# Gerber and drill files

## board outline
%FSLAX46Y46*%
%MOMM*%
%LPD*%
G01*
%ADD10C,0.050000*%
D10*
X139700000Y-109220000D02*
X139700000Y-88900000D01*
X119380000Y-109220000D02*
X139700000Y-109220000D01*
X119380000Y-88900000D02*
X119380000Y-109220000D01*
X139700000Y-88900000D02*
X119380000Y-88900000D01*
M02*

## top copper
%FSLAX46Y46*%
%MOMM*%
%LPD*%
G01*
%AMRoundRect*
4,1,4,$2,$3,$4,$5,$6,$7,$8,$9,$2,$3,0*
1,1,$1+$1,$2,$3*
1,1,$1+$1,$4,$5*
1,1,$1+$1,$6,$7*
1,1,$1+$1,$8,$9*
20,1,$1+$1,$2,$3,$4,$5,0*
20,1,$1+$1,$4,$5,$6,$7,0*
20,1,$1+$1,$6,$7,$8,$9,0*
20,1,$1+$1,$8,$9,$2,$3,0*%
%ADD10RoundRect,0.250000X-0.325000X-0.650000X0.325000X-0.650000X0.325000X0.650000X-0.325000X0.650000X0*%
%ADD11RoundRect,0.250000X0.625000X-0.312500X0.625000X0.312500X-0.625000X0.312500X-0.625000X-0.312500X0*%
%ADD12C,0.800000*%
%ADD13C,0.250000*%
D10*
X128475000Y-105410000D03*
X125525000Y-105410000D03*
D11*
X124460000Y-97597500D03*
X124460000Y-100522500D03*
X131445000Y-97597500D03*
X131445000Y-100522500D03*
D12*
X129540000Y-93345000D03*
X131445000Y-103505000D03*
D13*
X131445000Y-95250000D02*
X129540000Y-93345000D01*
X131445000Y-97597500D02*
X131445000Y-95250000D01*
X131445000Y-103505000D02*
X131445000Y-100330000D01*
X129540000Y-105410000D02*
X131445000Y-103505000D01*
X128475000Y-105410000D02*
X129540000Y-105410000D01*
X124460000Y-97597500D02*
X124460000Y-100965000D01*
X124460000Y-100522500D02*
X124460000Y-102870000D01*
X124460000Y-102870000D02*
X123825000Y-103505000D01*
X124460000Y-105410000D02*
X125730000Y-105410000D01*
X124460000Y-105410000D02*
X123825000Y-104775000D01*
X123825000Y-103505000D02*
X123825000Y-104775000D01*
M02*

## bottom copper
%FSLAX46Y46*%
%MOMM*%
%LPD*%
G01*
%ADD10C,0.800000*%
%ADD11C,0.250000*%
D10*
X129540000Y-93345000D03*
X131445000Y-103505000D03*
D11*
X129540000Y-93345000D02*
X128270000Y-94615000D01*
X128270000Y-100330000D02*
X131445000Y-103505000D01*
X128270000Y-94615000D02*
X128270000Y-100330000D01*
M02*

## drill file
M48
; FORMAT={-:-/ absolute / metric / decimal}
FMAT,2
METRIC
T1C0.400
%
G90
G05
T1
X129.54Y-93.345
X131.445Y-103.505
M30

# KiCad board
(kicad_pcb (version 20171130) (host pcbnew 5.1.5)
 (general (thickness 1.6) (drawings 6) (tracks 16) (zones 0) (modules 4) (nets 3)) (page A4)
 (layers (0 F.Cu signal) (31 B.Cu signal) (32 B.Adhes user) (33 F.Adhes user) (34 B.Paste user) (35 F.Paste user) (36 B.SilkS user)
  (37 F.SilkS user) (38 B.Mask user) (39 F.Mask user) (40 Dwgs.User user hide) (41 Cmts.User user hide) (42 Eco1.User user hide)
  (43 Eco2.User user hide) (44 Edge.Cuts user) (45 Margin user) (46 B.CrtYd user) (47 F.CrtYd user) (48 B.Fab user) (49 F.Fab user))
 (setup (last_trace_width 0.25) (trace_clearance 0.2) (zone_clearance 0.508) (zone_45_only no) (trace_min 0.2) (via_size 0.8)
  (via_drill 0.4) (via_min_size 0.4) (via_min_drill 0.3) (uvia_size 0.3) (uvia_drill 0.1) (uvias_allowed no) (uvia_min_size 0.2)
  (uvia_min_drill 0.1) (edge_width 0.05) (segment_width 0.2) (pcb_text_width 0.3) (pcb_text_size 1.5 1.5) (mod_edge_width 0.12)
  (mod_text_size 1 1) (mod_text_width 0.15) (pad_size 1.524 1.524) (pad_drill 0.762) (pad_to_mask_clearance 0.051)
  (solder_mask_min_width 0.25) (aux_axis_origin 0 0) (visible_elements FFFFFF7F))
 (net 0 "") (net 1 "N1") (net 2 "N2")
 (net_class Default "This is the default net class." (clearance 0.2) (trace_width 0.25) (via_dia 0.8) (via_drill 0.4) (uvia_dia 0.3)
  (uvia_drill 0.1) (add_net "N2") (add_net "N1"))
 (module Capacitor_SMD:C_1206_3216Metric (layer F.Cu) (at 127 105.41)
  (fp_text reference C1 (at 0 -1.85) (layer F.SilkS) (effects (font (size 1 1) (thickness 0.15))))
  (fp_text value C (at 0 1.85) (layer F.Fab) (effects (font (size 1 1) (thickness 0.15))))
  (pad 2 smd roundrect (at 1.475 0) (size 1.15 1.8) (layers F.Cu F.Paste F.Mask) (roundrect_rratio 0.217391) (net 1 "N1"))
  (pad 1 smd roundrect (at -1.475 0) (size 1.15 1.8) (layers F.Cu F.Paste F.Mask) (roundrect_rratio 0.217391) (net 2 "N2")))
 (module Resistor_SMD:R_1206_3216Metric (layer F.Cu) (at 124.46 99.06 90)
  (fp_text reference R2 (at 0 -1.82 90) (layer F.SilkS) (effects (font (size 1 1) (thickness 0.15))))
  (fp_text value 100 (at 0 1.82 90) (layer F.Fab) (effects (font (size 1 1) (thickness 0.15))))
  (pad 2 smd roundrect (at 1.4625 0 90) (size 1.125 1.75) (layers F.Cu F.Paste F.Mask) (roundrect_rratio 0.222222) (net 2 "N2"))
  (pad 1 smd roundrect (at -1.4625 0 90) (size 1.125 1.75) (layers F.Cu F.Paste F.Mask) (roundrect_rratio 0.222222) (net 2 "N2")))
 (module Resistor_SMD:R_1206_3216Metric (layer F.Cu) (at 131.445 99.06 90)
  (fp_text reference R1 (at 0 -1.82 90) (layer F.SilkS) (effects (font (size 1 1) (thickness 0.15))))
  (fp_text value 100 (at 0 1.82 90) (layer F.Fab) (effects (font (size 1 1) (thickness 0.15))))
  (pad 2 smd roundrect (at 1.4625 0 90) (size 1.125 1.75) (layers F.Cu F.Paste F.Mask) (roundrect_rratio 0.222222) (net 1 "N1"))
  (pad 1 smd roundrect (at -1.4625 0 90) (size 1.125 1.75) (layers F.Cu F.Paste F.Mask) (roundrect_rratio 0.222222) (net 1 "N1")))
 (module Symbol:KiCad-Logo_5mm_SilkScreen (layer F.Cu) (at 137.795 95.25 90)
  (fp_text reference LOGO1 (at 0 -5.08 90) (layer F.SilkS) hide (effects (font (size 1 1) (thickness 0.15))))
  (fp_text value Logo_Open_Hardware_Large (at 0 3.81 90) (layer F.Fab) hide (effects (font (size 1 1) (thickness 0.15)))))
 (gr_line (start 139.7 109.22) (end 139.7 88.9) (layer Edge.Cuts) (width 0.05))
 (gr_line (start 119.38 109.22) (end 139.7 109.22) (layer Edge.Cuts) (width 0.05))
 (gr_line (start 119.38 88.9) (end 119.38 109.22) (layer Edge.Cuts) (width 0.05))
 (gr_line (start 139.7 88.9) (end 119.38 88.9) (layer Edge.Cuts) (width 0.05))
 (via (at 129.54 93.345) (size 0.8) (drill 0.4) (layers F.Cu B.Cu) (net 1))
 (segment (start 131.445 95.25) (end 129.54 93.345) (width 0.25) (layer F.Cu) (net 1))
 (segment (start 131.445 97.5975) (end 131.445 95.25) (width 0.25) (layer F.Cu) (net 1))
 (segment (start 129.54 93.345) (end 128.27 94.615) (width 0.25) (layer B.Cu) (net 1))
 (via (at 131.445 103.505) (size 0.8) (drill 0.4) (layers F.Cu B.Cu) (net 1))
 (segment (start 128.27 100.33) (end 131.445 103.505) (width 0.25) (layer B.Cu) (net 1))
 (segment (start 128.27 94.615) (end 128.27 100.33) (width 0.25) (layer B.Cu) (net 1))
 (segment (start 131.445 103.505) (end 131.445 100.33) (width 0.25) (layer F.Cu) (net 1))
 (segment (start 129.54 105.41) (end 131.445 103.505) (width 0.25) (layer F.Cu) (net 1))
 (segment (start 128.475 105.41) (end 129.54 105.41) (width 0.25) (layer F.Cu) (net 1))
 (segment (start 124.46 97.5975) (end 124.46 100.965) (width 0.25) (layer F.Cu) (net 2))
 (segment (start 124.46 100.5225) (end 124.46 102.87) (width 0.25) (layer F.Cu) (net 2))
 (segment (start 124.46 102.87) (end 123.825 103.505) (width 0.25) (layer F.Cu) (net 2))
 (segment (start 124.46 105.41) (end 125.73 105.41) (width 0.25) (layer F.Cu) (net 2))
 (segment (start 124.46 105.41) (end 123.825 104.775) (width 0.25) (layer F.Cu) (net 2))
 (segment (start 123.825 103.505) (end 123.825 104.775) (width 0.25) (layer F.Cu) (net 2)))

